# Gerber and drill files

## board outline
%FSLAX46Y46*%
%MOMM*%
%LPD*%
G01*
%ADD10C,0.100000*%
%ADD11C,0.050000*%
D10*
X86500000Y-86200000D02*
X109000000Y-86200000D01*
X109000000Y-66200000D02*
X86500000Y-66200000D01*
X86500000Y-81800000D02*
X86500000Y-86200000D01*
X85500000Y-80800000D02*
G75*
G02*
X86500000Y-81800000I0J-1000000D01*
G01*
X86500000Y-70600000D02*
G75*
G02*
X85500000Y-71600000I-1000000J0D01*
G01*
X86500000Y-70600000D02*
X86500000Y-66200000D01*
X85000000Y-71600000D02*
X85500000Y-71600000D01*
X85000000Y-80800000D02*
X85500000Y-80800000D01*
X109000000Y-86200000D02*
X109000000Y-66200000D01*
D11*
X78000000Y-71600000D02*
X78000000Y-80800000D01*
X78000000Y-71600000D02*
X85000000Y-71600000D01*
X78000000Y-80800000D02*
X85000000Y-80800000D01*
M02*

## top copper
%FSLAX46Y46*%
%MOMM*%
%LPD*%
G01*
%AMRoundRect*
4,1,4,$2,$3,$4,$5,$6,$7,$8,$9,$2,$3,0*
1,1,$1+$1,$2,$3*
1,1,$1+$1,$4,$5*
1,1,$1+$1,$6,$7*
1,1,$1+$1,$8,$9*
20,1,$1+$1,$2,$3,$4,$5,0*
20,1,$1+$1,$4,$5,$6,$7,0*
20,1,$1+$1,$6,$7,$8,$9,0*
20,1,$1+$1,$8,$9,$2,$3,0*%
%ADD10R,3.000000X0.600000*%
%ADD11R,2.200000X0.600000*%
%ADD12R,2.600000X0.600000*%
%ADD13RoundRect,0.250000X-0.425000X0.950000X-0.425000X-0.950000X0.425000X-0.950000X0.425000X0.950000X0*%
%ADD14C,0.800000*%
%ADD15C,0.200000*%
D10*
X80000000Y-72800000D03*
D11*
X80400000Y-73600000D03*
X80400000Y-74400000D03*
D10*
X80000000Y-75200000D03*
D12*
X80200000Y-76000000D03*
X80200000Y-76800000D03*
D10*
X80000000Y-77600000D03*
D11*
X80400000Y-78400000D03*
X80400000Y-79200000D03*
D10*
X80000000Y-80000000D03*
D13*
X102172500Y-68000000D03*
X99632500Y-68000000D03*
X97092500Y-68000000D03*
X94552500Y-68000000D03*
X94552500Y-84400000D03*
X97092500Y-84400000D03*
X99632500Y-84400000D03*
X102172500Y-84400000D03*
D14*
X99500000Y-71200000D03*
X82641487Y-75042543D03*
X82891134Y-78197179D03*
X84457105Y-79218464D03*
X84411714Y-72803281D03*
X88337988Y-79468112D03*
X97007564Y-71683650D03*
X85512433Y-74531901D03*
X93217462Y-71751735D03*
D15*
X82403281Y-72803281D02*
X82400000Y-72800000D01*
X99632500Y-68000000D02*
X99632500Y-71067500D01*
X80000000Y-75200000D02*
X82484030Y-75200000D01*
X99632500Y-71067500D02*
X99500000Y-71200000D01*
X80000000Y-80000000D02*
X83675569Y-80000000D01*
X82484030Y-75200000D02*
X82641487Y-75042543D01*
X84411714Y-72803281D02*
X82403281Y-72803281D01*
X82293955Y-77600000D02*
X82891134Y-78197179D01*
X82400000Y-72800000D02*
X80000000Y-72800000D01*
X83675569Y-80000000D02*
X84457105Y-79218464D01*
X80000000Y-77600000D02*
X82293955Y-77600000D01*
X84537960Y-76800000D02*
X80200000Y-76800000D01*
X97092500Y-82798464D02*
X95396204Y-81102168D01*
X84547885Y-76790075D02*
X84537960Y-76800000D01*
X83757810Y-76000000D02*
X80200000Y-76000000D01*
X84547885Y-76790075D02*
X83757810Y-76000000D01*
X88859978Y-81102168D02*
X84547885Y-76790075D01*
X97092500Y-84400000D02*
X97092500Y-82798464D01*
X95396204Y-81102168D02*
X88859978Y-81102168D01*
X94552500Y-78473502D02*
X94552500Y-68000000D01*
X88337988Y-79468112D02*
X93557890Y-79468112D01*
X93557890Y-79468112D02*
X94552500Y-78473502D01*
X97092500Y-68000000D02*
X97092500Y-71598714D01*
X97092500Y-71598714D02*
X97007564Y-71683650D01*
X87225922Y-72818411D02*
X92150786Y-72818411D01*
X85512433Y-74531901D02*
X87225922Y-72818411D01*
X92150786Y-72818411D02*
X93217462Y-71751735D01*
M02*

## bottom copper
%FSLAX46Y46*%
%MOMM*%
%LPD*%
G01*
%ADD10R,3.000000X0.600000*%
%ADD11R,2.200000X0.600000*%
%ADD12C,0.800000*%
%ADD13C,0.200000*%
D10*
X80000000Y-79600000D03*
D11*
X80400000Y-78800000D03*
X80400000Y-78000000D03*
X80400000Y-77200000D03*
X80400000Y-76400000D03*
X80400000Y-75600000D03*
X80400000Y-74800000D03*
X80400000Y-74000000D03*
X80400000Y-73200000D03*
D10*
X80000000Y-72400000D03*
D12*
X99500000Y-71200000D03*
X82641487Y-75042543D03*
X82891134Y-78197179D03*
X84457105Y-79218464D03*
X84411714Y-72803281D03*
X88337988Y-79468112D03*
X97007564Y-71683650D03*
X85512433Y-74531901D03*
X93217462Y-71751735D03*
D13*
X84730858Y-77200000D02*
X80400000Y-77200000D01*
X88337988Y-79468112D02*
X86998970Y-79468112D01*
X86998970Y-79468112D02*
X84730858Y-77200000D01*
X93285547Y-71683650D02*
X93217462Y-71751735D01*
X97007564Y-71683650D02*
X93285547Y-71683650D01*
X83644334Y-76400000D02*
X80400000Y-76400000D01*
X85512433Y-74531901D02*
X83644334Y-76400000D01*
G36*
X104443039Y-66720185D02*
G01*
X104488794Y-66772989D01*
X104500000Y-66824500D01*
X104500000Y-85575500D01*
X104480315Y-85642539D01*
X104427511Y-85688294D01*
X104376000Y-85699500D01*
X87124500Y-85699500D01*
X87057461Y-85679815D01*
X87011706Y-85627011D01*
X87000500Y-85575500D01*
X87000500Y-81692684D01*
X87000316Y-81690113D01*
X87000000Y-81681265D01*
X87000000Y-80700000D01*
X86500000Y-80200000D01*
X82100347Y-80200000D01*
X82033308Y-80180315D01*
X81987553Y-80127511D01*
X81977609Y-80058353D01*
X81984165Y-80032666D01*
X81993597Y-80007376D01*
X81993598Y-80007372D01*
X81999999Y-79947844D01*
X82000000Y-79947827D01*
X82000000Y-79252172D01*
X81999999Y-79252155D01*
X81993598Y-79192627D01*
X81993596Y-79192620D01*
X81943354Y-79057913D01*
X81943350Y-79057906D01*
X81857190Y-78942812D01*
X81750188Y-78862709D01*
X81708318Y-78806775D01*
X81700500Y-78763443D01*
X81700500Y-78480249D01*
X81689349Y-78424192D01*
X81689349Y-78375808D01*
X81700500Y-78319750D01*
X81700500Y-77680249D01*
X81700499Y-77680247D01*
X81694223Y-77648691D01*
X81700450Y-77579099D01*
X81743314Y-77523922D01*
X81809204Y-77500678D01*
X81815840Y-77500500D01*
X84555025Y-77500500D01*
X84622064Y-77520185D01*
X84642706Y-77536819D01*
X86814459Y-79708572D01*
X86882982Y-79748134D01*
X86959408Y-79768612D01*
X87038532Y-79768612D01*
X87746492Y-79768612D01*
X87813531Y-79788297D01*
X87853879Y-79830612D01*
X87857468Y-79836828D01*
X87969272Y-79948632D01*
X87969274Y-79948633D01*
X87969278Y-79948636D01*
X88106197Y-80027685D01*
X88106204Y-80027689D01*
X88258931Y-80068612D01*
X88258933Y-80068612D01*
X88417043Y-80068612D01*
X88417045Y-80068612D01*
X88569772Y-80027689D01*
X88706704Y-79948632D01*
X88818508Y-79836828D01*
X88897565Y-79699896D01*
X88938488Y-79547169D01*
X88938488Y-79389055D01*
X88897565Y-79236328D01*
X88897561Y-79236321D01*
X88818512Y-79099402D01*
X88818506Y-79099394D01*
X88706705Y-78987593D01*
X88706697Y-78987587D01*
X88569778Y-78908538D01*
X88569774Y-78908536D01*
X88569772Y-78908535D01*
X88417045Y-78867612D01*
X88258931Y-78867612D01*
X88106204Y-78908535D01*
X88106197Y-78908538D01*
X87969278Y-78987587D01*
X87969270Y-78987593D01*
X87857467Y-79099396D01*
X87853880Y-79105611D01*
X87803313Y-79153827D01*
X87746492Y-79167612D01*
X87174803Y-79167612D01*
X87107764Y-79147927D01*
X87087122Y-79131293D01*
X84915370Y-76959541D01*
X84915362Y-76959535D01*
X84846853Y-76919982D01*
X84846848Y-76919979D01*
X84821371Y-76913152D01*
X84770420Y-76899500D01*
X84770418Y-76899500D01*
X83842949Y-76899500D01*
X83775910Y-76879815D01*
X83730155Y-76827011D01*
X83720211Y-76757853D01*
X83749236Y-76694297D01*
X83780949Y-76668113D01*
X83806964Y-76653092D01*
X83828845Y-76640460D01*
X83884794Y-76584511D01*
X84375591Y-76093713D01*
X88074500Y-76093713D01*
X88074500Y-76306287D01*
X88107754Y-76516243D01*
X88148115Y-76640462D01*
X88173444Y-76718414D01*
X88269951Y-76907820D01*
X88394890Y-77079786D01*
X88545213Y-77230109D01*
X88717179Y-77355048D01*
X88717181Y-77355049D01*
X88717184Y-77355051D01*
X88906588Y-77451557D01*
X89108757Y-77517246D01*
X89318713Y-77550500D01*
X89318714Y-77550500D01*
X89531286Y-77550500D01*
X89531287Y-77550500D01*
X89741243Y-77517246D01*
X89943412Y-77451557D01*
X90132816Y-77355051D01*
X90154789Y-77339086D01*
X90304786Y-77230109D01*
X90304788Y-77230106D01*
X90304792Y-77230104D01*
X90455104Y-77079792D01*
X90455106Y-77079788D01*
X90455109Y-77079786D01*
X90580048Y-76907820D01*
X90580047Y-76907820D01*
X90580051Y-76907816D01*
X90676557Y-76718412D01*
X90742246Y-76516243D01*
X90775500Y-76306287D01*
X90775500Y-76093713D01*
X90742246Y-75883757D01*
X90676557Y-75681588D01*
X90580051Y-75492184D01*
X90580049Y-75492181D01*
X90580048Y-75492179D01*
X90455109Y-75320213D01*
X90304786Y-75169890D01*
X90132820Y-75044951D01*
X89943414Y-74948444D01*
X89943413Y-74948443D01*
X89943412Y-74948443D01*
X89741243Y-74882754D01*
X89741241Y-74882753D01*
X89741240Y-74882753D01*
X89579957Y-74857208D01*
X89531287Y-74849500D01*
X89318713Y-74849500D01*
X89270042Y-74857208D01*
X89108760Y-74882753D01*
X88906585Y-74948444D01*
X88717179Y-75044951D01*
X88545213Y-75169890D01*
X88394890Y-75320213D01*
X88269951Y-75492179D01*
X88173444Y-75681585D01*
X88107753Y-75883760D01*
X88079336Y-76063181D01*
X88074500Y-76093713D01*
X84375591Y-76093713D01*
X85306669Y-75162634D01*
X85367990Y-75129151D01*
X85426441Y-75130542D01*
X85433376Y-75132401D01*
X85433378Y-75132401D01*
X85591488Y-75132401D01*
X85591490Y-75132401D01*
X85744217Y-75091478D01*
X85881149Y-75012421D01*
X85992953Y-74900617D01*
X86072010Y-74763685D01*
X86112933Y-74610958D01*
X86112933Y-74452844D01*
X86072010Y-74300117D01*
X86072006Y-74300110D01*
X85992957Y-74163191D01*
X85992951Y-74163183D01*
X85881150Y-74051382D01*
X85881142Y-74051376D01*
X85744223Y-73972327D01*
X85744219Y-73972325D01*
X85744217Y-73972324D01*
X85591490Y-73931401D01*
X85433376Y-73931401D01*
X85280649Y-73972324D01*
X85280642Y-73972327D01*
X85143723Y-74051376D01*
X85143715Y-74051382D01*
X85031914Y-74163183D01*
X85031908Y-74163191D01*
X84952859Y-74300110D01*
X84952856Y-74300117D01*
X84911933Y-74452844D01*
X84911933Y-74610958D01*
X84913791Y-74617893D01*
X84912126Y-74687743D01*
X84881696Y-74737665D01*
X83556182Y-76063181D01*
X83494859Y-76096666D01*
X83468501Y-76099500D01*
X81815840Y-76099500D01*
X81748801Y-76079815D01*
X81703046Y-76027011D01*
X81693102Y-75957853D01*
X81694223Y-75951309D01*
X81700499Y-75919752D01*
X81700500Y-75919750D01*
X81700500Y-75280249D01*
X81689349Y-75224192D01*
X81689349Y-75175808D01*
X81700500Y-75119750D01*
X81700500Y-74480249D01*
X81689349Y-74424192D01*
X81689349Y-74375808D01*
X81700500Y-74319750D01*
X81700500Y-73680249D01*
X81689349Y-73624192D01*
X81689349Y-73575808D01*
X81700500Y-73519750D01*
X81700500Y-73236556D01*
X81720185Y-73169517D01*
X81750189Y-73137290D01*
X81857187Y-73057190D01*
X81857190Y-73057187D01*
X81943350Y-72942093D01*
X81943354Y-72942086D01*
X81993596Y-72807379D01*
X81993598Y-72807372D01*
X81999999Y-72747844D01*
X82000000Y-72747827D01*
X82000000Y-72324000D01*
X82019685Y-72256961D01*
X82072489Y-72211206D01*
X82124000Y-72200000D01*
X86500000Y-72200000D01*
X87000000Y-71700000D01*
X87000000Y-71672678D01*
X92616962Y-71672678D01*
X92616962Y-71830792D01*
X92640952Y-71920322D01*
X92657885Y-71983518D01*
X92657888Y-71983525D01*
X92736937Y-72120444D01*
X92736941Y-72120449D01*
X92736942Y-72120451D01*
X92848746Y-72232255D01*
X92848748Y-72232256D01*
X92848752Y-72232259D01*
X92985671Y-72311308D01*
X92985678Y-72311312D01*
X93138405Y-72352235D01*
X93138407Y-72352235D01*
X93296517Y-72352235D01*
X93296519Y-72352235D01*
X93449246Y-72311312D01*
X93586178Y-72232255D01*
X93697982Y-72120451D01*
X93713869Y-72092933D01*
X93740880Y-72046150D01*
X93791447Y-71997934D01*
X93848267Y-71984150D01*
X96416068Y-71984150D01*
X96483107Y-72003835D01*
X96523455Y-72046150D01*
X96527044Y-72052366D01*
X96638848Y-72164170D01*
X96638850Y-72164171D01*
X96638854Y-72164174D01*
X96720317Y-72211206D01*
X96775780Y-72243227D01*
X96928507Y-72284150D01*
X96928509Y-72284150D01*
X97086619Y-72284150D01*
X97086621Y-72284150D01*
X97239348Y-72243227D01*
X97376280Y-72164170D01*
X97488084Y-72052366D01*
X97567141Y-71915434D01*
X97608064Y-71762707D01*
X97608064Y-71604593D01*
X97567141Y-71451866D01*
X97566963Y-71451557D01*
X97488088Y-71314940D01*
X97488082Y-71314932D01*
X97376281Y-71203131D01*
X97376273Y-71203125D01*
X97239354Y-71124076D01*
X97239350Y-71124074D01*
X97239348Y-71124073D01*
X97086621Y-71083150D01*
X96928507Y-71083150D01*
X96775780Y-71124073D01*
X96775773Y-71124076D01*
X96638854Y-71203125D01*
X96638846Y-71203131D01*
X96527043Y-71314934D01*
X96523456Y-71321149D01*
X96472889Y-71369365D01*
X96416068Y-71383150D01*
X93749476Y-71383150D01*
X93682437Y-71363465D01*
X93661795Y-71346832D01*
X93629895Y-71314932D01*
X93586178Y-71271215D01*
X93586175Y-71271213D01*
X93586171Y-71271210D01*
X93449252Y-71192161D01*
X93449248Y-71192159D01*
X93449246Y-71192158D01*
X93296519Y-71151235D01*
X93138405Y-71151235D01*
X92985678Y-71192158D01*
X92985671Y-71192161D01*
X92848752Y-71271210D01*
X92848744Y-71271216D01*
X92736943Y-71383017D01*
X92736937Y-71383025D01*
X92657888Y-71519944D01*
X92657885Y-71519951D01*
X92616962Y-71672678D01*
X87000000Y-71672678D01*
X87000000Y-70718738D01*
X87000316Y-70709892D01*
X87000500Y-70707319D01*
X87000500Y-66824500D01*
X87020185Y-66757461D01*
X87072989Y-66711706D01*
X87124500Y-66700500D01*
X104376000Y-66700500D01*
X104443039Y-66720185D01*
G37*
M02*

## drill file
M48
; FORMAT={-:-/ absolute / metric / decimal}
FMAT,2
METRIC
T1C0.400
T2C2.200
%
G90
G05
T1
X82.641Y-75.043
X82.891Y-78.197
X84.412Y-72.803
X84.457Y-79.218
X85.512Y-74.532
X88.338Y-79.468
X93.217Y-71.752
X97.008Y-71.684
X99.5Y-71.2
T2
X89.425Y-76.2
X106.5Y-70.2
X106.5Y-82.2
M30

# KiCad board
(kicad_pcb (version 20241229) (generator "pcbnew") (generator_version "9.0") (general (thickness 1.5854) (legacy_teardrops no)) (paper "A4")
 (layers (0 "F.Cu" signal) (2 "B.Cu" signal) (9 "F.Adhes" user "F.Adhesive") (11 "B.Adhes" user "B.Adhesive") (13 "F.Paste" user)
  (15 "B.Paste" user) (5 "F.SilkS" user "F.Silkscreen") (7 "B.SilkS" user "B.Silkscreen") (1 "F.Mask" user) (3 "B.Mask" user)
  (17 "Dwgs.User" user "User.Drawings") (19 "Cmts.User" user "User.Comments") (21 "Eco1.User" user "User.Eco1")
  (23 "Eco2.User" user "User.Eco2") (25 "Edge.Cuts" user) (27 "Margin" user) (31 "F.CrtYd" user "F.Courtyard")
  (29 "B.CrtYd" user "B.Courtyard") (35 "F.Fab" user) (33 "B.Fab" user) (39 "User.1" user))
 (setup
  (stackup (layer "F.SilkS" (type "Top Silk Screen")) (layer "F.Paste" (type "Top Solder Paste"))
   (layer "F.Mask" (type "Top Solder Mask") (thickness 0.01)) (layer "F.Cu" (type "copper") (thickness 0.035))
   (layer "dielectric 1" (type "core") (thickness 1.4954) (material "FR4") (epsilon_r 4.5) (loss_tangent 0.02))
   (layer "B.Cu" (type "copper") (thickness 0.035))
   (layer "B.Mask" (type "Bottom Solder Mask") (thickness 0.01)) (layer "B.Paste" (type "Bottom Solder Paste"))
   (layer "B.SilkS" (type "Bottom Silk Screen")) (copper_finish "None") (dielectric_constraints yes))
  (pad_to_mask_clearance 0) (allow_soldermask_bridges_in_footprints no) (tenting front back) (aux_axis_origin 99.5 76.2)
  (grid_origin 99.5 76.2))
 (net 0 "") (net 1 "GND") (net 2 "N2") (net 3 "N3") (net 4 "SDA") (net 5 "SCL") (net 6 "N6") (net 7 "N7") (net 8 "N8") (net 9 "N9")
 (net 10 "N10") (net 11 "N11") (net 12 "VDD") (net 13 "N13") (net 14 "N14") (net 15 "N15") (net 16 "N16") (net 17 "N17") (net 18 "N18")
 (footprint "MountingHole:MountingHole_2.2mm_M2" (layer "F.Cu") (at 106.5 82.2)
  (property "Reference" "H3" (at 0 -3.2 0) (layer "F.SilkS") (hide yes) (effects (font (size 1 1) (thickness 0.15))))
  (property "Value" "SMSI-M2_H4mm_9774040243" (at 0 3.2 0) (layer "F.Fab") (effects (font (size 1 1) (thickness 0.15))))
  (pad "" np_thru_hole circle (at 0 0) (size 2.2 2.2) (drill 2.2) (layers "*.Cu" "*.Mask")))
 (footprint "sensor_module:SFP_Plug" (layer "F.Cu") (at 81.5 76.2 180)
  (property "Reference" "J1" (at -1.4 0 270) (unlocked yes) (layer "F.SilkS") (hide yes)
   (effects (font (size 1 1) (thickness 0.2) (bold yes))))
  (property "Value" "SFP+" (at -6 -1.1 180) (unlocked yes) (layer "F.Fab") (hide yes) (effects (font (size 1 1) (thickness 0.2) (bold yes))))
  (fp_line (start 3.5 4.6) (end 3.5 -4.6) (stroke (width 0.05) (type default)) (layer "Edge.Cuts"))
  (fp_line (start 3.5 4.6) (end -3.5 4.6) (stroke (width 0.05) (type solid)) (layer "Edge.Cuts"))
  (fp_line (start 3.5 -4.6) (end -3.5 -4.6) (stroke (width 0.05) (type solid)) (layer "Edge.Cuts"))
  (pad "1" smd rect (at 1.5 -3.4 180) (size 3 0.6) (layers "B.Cu" "B.Mask") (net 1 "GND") (thermal_bridge_angle 45))
  (pad "2" smd rect (at 1.1 -2.6 180) (size 2.2 0.6) (layers "B.Cu" "B.Mask") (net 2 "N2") (thermal_bridge_angle 45))
  (pad "3" smd rect (at 1.1 -1.8 180) (size 2.2 0.6) (layers "B.Cu" "B.Mask") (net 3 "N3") (thermal_bridge_angle 45))
  (pad "4" smd rect (at 1.1 -1 180) (size 2.2 0.6) (layers "B.Cu" "B.Mask") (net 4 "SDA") (thermal_bridge_angle 45))
  (pad "5" smd rect (at 1.1 -0.2 180) (size 2.2 0.6) (layers "B.Cu" "B.Mask") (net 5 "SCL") (thermal_bridge_angle 45))
  (pad "6" smd rect (at 1.1 0.6 180) (size 2.2 0.6) (layers "B.Cu" "B.Mask") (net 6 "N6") (thermal_bridge_angle 45))
  (pad "7" smd rect (at 1.1 1.4 180) (size 2.2 0.6) (layers "B.Cu" "B.Mask") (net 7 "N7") (thermal_bridge_angle 45))
  (pad "8" smd rect (at 1.1 2.2 180) (size 2.2 0.6) (layers "B.Cu" "B.Mask") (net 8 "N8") (thermal_bridge_angle 45))
  (pad "9" smd rect (at 1.1 3 180) (size 2.2 0.6) (layers "B.Cu" "B.Mask") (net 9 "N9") (thermal_bridge_angle 45))
  (pad "10" smd rect (at 1.5 3.8 180) (size 3 0.6) (layers "B.Cu" "B.Mask") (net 1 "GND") (thermal_bridge_angle 45))
  (pad "11" smd rect (at 1.5 3.4 180) (size 3 0.6) (layers "F.Cu" "F.Mask") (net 1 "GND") (thermal_bridge_angle 45))
  (pad "12" smd rect (at 1.1 2.6 180) (size 2.2 0.6) (layers "F.Cu" "F.Mask") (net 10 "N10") (thermal_bridge_angle 45))
  (pad "13" smd rect (at 1.1 1.8 180) (size 2.2 0.6) (layers "F.Cu" "F.Mask") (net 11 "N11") (thermal_bridge_angle 45))
  (pad "14" smd rect (at 1.5 1 180) (size 3 0.6) (layers "F.Cu" "F.Mask") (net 1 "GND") (thermal_bridge_angle 45))
  (pad "15" smd rect (at 1.3 0.2 180) (size 2.6 0.6) (layers "F.Cu" "F.Mask") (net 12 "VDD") (thermal_bridge_angle 45))
  (pad "16" smd rect (at 1.3 -0.6 180) (size 2.6 0.6) (layers "F.Cu" "F.Mask") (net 12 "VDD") (thermal_bridge_angle 45))
  (pad "17" smd rect (at 1.5 -1.4 180) (size 3 0.6) (layers "F.Cu" "F.Mask") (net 1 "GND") (thermal_bridge_angle 45))
  (pad "18" smd rect (at 1.1 -2.2 180) (size 2.2 0.6) (layers "F.Cu" "F.Mask") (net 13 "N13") (thermal_bridge_angle 45))
  (pad "19" smd rect (at 1.1 -3 180) (size 2.2 0.6) (layers "F.Cu" "F.Mask") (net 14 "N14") (thermal_bridge_angle 45))
  (pad "20" smd rect (at 1.5 -3.8 180) (size 3 0.6) (layers "F.Cu" "F.Mask") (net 1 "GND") (thermal_bridge_angle 45)))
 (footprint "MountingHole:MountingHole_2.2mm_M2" (layer "F.Cu") (at 106.5 70.2)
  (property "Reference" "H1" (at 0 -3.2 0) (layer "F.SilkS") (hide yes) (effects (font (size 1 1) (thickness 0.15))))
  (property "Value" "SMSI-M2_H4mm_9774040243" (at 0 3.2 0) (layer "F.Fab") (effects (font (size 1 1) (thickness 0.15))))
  (pad "" np_thru_hole circle (at 0 0) (size 2.2 2.2) (drill 2.2) (layers "*.Cu" "*.Mask")))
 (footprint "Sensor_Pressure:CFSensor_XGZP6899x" (layer "F.Cu") (at 98.3625 76.2 -90)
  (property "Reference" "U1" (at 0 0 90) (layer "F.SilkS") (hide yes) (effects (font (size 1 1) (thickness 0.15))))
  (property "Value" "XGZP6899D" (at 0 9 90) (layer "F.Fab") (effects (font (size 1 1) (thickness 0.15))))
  (pad "1" smd roundrect (at -8.2 -3.81 270) (size 2.4 1.35) (layers "F.Cu" "F.Mask" "F.Paste") (roundrect_rratio 0.185185) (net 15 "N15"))
  (pad "2" smd roundrect (at -8.2 -1.27 270) (size 2.4 1.35) (layers "F.Cu" "F.Mask" "F.Paste") (roundrect_rratio 0.185185) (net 1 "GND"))
  (pad "3" smd roundrect (at -8.2 1.27 270) (size 2.4 1.35) (layers "F.Cu" "F.Mask" "F.Paste") (roundrect_rratio 0.185185) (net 5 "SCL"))
  (pad "4" smd roundrect (at -8.2 3.81 270) (size 2.4 1.35) (layers "F.Cu" "F.Mask" "F.Paste") (roundrect_rratio 0.185185) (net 4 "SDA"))
  (pad "5" smd roundrect (at 8.2 3.81 270) (size 2.4 1.35) (layers "F.Cu" "F.Mask" "F.Paste") (roundrect_rratio 0.185185) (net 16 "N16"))
  (pad "6" smd roundrect (at 8.2 1.27 270) (size 2.4 1.35) (layers "F.Cu" "F.Mask" "F.Paste") (roundrect_rratio 0.185185) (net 12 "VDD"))
  (pad "7" smd roundrect (at 8.2 -1.27 270) (size 2.4 1.35) (layers "F.Cu" "F.Mask" "F.Paste") (roundrect_rratio 0.185185) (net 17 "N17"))
  (pad "8" smd roundrect (at 8.2 -3.81 270) (size 2.4 1.35) (layers "F.Cu" "F.Mask" "F.Paste") (roundrect_rratio 0.185185) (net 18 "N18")))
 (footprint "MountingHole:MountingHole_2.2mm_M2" (layer "F.Cu") (at 89.425 76.2)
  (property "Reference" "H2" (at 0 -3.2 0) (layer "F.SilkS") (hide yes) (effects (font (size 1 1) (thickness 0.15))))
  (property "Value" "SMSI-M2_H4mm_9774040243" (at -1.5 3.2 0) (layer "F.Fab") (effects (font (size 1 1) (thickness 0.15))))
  (pad "" np_thru_hole circle (at 0 0) (size 2.2 2.2) (drill 2.2) (layers "*.Cu" "*.Mask")))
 (gr_line (start 86.5 86.2) (end 109 86.2) (stroke (width 0.1) (type default)) (layer "Edge.Cuts"))
 (gr_line (start 109 66.2) (end 86.5 66.2) (stroke (width 0.1) (type default)) (layer "Edge.Cuts"))
 (gr_line (start 86.5 81.8) (end 86.5 86.2) (stroke (width 0.1) (type default)) (layer "Edge.Cuts"))
 (gr_arc (start 85.5 80.8) (mid 86.207107 81.092893) (end 86.5 81.8) (stroke (width 0.1) (type default)) (layer "Edge.Cuts"))
 (gr_arc (start 86.5 70.6) (mid 86.207107 71.307107) (end 85.5 71.6) (stroke (width 0.1) (type default)) (layer "Edge.Cuts"))
 (gr_line (start 86.5 70.6) (end 86.5 66.2) (stroke (width 0.1) (type default)) (layer "Edge.Cuts"))
 (gr_line (start 85 71.6) (end 85.5 71.6) (stroke (width 0.1) (type default)) (layer "Edge.Cuts"))
 (gr_line (start 85 80.8) (end 85.5 80.8) (stroke (width 0.1) (type default)) (layer "Edge.Cuts"))
 (gr_line (start 109 86.2) (end 109 66.2) (stroke (width 0.1) (type default)) (layer "Edge.Cuts"))
 (segment (start 82.403281 72.803281) (end 82.4 72.8) (width 0.2) (layer "F.Cu") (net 1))
 (segment (start 99.6325 68) (end 99.6325 71.0675) (width 0.2) (layer "F.Cu") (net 1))
 (segment (start 80 75.2) (end 82.48403 75.2) (width 0.2) (layer "F.Cu") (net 1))
 (segment (start 99.6325 71.0675) (end 99.5 71.2) (width 0.2) (layer "F.Cu") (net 1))
 (segment (start 80 80) (end 83.675569 80) (width 0.2) (layer "F.Cu") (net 1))
 (segment (start 82.48403 75.2) (end 82.641487 75.042543) (width 0.2) (layer "F.Cu") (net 1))
 (segment (start 84.411714 72.803281) (end 82.403281 72.803281) (width 0.2) (layer "F.Cu") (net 1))
 (segment (start 82.293955 77.6) (end 82.891134 78.197179) (width 0.2) (layer "F.Cu") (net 1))
 (segment (start 82.4 72.8) (end 80 72.8) (width 0.2) (layer "F.Cu") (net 1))
 (segment (start 83.675569 80) (end 84.457105 79.218464) (width 0.2) (layer "F.Cu") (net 1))
 (segment (start 80 77.6) (end 82.293955 77.6) (width 0.2) (layer "F.Cu") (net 1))
 (via (at 99.5 71.2) (size 0.8) (drill 0.4) (layers "F.Cu" "B.Cu") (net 1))
 (via (at 82.641487 75.042543) (size 0.8) (drill 0.4) (layers "F.Cu" "B.Cu") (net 1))
 (via (at 82.891134 78.197179) (size 0.8) (drill 0.4) (layers "F.Cu" "B.Cu") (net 1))
 (via (at 84.457105 79.218464) (size 0.8) (drill 0.4) (layers "F.Cu" "B.Cu") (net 1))
 (via (at 84.411714 72.803281) (size 0.8) (drill 0.4) (layers "F.Cu" "B.Cu") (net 1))
 (segment (start 84.53796 76.8) (end 80.2 76.8) (width 0.2) (layer "F.Cu") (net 12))
 (segment (start 97.0925 82.798464) (end 95.396204 81.102168) (width 0.2) (layer "F.Cu") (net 12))
 (segment (start 84.547885 76.790075) (end 84.53796 76.8) (width 0.2) (layer "F.Cu") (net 12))
 (segment (start 83.75781 76) (end 80.2 76) (width 0.2) (layer "F.Cu") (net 12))
 (segment (start 84.547885 76.790075) (end 83.75781 76) (width 0.2) (layer "F.Cu") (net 12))
 (segment (start 88.859978 81.102168) (end 84.547885 76.790075) (width 0.2) (layer "F.Cu") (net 12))
 (segment (start 97.0925 84.4) (end 97.0925 82.798464) (width 0.2) (layer "F.Cu") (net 12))
 (segment (start 95.396204 81.102168) (end 88.859978 81.102168) (width 0.2) (layer "F.Cu") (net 12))
 (segment (start 94.5525 78.473502) (end 94.5525 68) (width 0.2) (layer "F.Cu") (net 4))
 (segment (start 88.337988 79.468112) (end 93.55789 79.468112) (width 0.2) (layer "F.Cu") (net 4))
 (segment (start 93.55789 79.468112) (end 94.5525 78.473502) (width 0.2) (layer "F.Cu") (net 4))
 (via (at 88.337988 79.468112) (size 0.8) (drill 0.4) (layers "F.Cu" "B.Cu") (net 4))
 (segment (start 84.730858 77.2) (end 80.4 77.2) (width 0.2) (layer "B.Cu") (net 4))
 (segment (start 88.337988 79.468112) (end 86.99897 79.468112) (width 0.2) (layer "B.Cu") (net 4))
 (segment (start 86.99897 79.468112) (end 84.730858 77.2) (width 0.2) (layer "B.Cu") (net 4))
 (segment (start 97.0925 68) (end 97.0925 71.598714) (width 0.2) (layer "F.Cu") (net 5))
 (segment (start 97.0925 71.598714) (end 97.007564 71.68365) (width 0.2) (layer "F.Cu") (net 5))
 (segment (start 87.225922 72.818411) (end 92.150786 72.818411) (width 0.2) (layer "F.Cu") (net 5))
 (segment (start 85.512433 74.531901) (end 87.225922 72.818411) (width 0.2) (layer "F.Cu") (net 5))
 (segment (start 92.150786 72.818411) (end 93.217462 71.751735) (width 0.2) (layer "F.Cu") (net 5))
 (via (at 97.007564 71.68365) (size 0.8) (drill 0.4) (layers "F.Cu" "B.Cu") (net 5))
 (via (at 85.512433 74.531901) (size 0.8) (drill 0.4) (layers "F.Cu" "B.Cu") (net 5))
 (via (at 93.217462 71.751735) (size 0.8) (drill 0.4) (layers "F.Cu" "B.Cu") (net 5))
 (segment (start 93.285547 71.68365) (end 93.217462 71.751735) (width 0.2) (layer "B.Cu") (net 5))
 (segment (start 97.007564 71.68365) (end 93.285547 71.68365) (width 0.2) (layer "B.Cu") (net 5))
 (segment (start 83.644334 76.4) (end 80.4 76.4) (width 0.2) (layer "B.Cu") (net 5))
 (segment (start 85.512433 74.531901) (end 83.644334 76.4) (width 0.2) (layer "B.Cu") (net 5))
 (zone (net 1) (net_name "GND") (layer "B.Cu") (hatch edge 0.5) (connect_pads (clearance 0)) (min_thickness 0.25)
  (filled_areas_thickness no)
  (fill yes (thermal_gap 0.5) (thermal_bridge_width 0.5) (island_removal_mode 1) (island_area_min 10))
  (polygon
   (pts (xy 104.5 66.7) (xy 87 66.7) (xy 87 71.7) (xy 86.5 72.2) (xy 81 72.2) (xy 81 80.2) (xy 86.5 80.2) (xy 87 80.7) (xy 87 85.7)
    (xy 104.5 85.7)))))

